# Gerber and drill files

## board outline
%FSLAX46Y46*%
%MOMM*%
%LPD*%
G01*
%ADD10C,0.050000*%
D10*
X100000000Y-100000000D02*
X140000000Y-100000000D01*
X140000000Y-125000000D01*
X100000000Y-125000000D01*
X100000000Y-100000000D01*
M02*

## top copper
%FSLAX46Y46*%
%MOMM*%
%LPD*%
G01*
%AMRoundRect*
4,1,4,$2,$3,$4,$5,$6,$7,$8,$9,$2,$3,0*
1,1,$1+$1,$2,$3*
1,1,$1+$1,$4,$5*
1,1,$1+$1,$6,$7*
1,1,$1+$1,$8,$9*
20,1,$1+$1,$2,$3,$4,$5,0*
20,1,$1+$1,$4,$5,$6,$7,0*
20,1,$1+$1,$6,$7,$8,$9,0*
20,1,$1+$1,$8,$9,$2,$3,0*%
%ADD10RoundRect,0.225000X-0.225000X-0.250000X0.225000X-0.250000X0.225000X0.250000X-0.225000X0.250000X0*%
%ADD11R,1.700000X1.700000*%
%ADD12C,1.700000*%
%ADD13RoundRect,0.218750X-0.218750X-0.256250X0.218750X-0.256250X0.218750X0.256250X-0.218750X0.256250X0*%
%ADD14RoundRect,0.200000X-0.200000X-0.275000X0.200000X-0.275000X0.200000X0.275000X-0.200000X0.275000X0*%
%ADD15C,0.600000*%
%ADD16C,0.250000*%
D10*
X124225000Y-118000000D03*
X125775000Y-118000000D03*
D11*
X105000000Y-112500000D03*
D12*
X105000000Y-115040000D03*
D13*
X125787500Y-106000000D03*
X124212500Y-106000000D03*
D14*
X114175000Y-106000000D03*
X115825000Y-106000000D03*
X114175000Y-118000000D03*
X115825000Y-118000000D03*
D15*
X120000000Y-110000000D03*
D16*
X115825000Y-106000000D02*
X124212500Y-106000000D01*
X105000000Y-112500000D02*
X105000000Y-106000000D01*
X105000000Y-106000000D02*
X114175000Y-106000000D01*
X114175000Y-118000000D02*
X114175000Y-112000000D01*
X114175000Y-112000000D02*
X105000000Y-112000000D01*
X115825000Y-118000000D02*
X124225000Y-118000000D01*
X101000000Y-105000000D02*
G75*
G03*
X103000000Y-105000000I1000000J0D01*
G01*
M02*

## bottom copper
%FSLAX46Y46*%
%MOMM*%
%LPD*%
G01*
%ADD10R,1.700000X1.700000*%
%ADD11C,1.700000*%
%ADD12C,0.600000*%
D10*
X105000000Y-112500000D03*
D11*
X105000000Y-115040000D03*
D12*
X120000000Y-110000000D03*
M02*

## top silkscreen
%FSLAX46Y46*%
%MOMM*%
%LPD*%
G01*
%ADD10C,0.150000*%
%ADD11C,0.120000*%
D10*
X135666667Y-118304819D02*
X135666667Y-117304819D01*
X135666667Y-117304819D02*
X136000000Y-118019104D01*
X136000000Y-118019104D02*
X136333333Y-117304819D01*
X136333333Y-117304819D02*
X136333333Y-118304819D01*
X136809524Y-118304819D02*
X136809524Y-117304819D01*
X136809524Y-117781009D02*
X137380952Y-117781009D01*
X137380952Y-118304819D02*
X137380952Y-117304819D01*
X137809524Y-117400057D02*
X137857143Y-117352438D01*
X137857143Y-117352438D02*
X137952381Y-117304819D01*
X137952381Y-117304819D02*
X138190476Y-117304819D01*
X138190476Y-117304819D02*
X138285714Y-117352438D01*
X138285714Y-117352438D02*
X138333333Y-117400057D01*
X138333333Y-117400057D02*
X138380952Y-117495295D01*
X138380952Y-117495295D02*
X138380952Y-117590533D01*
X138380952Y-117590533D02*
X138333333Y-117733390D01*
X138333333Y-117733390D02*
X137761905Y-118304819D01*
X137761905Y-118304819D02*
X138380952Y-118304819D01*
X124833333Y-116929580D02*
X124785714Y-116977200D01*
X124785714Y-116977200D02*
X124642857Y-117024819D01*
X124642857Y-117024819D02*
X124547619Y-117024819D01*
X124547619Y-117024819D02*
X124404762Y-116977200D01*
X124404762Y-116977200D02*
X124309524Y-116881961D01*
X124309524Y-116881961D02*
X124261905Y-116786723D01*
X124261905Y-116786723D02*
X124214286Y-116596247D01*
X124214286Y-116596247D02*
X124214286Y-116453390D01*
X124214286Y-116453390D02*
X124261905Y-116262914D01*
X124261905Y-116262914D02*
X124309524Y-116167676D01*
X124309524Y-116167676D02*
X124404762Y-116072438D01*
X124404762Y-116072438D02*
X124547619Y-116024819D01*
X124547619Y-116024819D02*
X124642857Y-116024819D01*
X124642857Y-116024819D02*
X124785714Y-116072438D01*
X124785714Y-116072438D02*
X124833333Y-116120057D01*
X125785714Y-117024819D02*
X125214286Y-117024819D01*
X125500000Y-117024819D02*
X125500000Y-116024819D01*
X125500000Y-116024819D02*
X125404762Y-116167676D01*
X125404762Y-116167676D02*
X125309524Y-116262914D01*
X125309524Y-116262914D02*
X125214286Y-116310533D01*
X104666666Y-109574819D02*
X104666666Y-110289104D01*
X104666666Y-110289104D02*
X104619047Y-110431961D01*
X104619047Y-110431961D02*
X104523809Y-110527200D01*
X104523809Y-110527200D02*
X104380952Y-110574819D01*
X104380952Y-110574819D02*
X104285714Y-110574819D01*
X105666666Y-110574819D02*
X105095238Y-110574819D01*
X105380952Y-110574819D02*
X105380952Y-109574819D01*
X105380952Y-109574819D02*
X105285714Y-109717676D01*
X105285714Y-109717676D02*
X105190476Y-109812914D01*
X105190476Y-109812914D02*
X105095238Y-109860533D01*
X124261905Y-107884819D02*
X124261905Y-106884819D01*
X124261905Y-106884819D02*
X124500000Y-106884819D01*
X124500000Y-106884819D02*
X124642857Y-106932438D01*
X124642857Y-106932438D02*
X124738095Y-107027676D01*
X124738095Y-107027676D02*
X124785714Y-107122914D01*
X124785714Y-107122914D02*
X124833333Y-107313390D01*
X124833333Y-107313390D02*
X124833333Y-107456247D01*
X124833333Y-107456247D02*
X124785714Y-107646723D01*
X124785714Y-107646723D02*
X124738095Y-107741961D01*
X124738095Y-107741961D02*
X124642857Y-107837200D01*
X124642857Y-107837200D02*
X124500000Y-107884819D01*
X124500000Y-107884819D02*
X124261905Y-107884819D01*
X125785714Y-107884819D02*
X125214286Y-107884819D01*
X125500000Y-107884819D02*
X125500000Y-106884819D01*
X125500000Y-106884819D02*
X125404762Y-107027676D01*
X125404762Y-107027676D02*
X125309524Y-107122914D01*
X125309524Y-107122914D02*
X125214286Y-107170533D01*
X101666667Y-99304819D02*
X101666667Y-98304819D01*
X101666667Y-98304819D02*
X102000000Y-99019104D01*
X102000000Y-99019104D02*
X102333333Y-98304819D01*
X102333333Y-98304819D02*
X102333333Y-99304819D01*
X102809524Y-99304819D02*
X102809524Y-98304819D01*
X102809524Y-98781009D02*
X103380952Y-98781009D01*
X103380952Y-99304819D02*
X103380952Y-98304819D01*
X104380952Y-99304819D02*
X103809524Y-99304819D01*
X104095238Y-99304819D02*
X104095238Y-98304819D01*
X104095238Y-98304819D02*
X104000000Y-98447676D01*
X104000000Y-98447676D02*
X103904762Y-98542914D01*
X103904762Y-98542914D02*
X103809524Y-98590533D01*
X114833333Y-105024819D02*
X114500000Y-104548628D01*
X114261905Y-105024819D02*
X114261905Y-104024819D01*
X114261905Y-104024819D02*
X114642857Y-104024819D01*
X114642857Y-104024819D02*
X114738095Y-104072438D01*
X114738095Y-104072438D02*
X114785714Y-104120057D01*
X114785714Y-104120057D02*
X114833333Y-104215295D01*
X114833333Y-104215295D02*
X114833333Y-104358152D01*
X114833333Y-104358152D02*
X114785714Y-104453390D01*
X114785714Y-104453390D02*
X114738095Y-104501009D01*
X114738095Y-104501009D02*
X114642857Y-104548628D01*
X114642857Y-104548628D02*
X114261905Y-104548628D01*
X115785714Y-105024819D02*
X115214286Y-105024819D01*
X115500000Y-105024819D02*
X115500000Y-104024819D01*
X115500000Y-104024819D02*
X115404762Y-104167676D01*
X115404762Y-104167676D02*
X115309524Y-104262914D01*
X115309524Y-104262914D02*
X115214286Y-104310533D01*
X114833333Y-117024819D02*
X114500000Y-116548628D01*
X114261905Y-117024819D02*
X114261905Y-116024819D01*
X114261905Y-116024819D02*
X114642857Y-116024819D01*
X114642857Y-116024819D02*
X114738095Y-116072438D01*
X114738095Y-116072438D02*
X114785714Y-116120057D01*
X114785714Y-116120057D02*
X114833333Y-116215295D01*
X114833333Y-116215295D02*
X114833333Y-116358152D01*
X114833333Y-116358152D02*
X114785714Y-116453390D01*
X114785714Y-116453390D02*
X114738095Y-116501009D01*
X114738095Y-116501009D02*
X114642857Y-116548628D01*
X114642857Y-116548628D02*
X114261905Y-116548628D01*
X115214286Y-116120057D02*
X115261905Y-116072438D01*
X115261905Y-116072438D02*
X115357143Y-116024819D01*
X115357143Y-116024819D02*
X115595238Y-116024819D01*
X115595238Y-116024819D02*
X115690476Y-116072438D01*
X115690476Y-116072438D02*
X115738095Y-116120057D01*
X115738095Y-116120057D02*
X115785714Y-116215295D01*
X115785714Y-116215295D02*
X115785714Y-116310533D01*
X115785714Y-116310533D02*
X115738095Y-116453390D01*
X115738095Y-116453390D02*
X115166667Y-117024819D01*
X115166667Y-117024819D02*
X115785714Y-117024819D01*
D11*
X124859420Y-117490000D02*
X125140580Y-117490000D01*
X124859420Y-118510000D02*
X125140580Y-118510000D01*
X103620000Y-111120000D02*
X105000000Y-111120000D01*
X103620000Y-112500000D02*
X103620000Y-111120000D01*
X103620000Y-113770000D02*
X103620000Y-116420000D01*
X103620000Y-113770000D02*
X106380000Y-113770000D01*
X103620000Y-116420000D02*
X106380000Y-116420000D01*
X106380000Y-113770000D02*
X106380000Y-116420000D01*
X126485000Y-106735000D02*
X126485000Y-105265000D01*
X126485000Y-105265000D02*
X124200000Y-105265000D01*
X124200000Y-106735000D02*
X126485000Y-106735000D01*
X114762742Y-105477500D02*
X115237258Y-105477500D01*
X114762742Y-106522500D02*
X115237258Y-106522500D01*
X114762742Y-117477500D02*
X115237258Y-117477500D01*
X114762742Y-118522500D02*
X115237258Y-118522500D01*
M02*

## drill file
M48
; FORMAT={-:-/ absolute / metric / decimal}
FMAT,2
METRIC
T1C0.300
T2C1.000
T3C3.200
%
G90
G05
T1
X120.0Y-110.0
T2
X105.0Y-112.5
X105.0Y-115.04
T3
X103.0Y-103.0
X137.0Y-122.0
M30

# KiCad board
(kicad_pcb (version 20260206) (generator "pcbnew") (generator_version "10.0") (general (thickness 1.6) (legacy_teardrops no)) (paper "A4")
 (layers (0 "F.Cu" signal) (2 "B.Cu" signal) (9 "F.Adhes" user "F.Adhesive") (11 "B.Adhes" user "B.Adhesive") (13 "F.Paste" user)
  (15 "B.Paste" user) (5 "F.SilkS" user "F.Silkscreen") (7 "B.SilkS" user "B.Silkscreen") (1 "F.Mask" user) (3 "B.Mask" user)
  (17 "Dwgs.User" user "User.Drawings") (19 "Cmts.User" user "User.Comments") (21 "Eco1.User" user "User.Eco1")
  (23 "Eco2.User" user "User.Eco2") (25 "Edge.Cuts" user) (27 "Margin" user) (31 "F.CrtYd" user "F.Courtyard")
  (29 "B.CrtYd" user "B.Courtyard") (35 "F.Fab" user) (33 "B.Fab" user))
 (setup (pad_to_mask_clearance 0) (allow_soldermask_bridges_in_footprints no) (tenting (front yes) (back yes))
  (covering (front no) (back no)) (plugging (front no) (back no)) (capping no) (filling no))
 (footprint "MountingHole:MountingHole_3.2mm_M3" (layer "F.Cu") (at 137 122)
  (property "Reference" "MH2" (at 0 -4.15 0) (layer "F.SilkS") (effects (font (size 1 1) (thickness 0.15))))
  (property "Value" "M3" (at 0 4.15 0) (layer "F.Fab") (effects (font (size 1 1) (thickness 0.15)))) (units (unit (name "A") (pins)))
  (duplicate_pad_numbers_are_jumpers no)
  (pad "" np_thru_hole circle (at 0 0) (size 3.2 3.2) (drill 3.2) (layers "*.Cu" "*.Mask")))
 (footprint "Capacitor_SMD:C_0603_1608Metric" (layer "F.Cu") (at 125 118)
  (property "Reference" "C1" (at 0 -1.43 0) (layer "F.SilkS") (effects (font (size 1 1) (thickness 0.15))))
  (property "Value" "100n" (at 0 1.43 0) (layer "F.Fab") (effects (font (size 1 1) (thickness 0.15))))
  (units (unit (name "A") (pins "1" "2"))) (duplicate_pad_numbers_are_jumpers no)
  (fp_line (start -0.14058 -0.51) (end 0.14058 -0.51) (stroke (width 0.12) (type solid)) (layer "F.SilkS"))
  (fp_line (start -0.14058 0.51) (end 0.14058 0.51) (stroke (width 0.12) (type solid)) (layer "F.SilkS"))
  (pad "1" smd roundrect (at -0.775 0) (size 0.9 0.95) (layers "F.Cu" "F.Mask" "F.Paste") (roundrect_rratio 0.25) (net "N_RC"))
  (pad "2" smd roundrect (at 0.775 0) (size 0.9 0.95) (layers "F.Cu" "F.Mask" "F.Paste") (roundrect_rratio 0.25) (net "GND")))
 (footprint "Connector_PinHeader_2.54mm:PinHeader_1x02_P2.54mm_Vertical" (layer "F.Cu") (at 105 112.5)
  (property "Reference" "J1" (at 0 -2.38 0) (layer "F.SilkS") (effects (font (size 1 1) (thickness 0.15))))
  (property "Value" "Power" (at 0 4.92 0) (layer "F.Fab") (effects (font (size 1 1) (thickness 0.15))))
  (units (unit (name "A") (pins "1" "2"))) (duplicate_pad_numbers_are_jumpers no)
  (fp_line (start -1.38 -1.38) (end 0 -1.38) (stroke (width 0.12) (type solid)) (layer "F.SilkS"))
  (fp_line (start -1.38 0) (end -1.38 -1.38) (stroke (width 0.12) (type solid)) (layer "F.SilkS"))
  (fp_line (start -1.38 1.27) (end -1.38 3.92) (stroke (width 0.12) (type solid)) (layer "F.SilkS"))
  (fp_line (start -1.38 1.27) (end 1.38 1.27) (stroke (width 0.12) (type solid)) (layer "F.SilkS"))
  (fp_line (start -1.38 3.92) (end 1.38 3.92) (stroke (width 0.12) (type solid)) (layer "F.SilkS"))
  (fp_line (start 1.38 1.27) (end 1.38 3.92) (stroke (width 0.12) (type solid)) (layer "F.SilkS"))
  (pad "1" thru_hole rect (at 0 0) (size 1.7 1.7) (drill 1) (layers "*.Cu" "*.Mask") (remove_unused_layers no) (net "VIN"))
  (pad "2" thru_hole circle (at 0 2.54) (size 1.7 1.7) (drill 1) (layers "*.Cu" "*.Mask") (remove_unused_layers no) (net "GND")))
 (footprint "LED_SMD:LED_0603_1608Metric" (layer "F.Cu") (at 125 106 180)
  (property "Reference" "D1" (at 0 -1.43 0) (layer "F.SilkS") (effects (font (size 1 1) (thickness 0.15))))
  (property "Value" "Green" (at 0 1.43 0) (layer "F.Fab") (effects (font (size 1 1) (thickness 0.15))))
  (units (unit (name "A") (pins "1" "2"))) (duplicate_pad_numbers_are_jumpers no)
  (fp_line (start -1.485 -0.735) (end -1.485 0.735) (stroke (width 0.12) (type solid)) (layer "F.SilkS"))
  (fp_line (start -1.485 0.735) (end 0.8 0.735) (stroke (width 0.12) (type solid)) (layer "F.SilkS"))
  (fp_line (start 0.8 -0.735) (end -1.485 -0.735) (stroke (width 0.12) (type solid)) (layer "F.SilkS"))
  (pad "1" smd roundrect (at -0.7875 0) (size 0.875 0.95) (layers "F.Cu" "F.Mask" "F.Paste") (roundrect_rratio 0.25) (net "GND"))
  (pad "2" smd roundrect (at 0.7875 0) (size 0.875 0.95) (layers "F.Cu" "F.Mask" "F.Paste") (roundrect_rratio 0.25) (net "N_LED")))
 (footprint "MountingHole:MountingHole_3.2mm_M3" (layer "F.Cu") (at 103 103)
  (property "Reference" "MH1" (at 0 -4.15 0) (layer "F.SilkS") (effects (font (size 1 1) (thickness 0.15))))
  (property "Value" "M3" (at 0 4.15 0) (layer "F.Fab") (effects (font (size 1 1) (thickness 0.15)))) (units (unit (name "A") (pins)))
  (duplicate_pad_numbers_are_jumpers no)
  (pad "" np_thru_hole circle (at 0 0) (size 3.2 3.2) (drill 3.2) (layers "*.Cu" "*.Mask")))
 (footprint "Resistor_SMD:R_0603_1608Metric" (layer "F.Cu") (at 115 106)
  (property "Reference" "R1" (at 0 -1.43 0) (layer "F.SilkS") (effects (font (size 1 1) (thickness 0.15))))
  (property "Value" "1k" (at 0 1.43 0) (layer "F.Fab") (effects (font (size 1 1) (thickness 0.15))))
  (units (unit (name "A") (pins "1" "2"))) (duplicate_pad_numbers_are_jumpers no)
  (fp_line (start -0.237258 -0.5225) (end 0.237258 -0.5225) (stroke (width 0.12) (type solid)) (layer "F.SilkS"))
  (fp_line (start -0.237258 0.5225) (end 0.237258 0.5225) (stroke (width 0.12) (type solid)) (layer "F.SilkS"))
  (pad "1" smd roundrect (at -0.825 0) (size 0.8 0.95) (layers "F.Cu" "F.Mask" "F.Paste") (roundrect_rratio 0.25) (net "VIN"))
  (pad "2" smd roundrect (at 0.825 0) (size 0.8 0.95) (layers "F.Cu" "F.Mask" "F.Paste") (roundrect_rratio 0.25) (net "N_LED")))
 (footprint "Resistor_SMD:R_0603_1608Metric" (layer "F.Cu") (at 115 118)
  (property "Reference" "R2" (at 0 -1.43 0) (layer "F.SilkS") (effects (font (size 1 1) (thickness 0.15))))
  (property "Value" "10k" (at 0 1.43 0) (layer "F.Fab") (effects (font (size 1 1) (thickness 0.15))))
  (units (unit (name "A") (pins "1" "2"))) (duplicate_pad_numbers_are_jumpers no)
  (fp_line (start -0.237258 -0.5225) (end 0.237258 -0.5225) (stroke (width 0.12) (type solid)) (layer "F.SilkS"))
  (fp_line (start -0.237258 0.5225) (end 0.237258 0.5225) (stroke (width 0.12) (type solid)) (layer "F.SilkS"))
  (pad "1" smd roundrect (at -0.825 0) (size 0.8 0.95) (layers "F.Cu" "F.Mask" "F.Paste") (roundrect_rratio 0.25) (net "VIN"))
  (pad "2" smd roundrect (at 0.825 0) (size 0.8 0.95) (layers "F.Cu" "F.Mask" "F.Paste") (roundrect_rratio 0.25) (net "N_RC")))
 (gr_rect (start 100 100) (end 140 125) (stroke (width 0.05) (type default)) (fill no) (layer "Edge.Cuts"))
 (segment (start 115.825 106) (end 124.2125 106) (width 0.25) (layer "F.Cu") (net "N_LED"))
 (segment (start 105 112.5) (end 105 106) (width 0.25) (layer "F.Cu") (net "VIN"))
 (segment (start 105 106) (end 114.175 106) (width 0.25) (layer "F.Cu") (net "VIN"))
 (segment (start 114.175 118) (end 114.175 112) (width 0.25) (layer "F.Cu") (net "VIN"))
 (segment (start 114.175 112) (end 105 112) (width 0.25) (layer "F.Cu") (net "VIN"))
 (segment (start 115.825 118) (end 124.225 118) (width 0.25) (layer "F.Cu") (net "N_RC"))
 (via (at 120 110) (size 0.6) (drill 0.3) (layers "F.Cu" "B.Cu") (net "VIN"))
 (arc (start 101 105) (mid 102 106) (end 103 105) (width 0.25) (layer "F.Cu") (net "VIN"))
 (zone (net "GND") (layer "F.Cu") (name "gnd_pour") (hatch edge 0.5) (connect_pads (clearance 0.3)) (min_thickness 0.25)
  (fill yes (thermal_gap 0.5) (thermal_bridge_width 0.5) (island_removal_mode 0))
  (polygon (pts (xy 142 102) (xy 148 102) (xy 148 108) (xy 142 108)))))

